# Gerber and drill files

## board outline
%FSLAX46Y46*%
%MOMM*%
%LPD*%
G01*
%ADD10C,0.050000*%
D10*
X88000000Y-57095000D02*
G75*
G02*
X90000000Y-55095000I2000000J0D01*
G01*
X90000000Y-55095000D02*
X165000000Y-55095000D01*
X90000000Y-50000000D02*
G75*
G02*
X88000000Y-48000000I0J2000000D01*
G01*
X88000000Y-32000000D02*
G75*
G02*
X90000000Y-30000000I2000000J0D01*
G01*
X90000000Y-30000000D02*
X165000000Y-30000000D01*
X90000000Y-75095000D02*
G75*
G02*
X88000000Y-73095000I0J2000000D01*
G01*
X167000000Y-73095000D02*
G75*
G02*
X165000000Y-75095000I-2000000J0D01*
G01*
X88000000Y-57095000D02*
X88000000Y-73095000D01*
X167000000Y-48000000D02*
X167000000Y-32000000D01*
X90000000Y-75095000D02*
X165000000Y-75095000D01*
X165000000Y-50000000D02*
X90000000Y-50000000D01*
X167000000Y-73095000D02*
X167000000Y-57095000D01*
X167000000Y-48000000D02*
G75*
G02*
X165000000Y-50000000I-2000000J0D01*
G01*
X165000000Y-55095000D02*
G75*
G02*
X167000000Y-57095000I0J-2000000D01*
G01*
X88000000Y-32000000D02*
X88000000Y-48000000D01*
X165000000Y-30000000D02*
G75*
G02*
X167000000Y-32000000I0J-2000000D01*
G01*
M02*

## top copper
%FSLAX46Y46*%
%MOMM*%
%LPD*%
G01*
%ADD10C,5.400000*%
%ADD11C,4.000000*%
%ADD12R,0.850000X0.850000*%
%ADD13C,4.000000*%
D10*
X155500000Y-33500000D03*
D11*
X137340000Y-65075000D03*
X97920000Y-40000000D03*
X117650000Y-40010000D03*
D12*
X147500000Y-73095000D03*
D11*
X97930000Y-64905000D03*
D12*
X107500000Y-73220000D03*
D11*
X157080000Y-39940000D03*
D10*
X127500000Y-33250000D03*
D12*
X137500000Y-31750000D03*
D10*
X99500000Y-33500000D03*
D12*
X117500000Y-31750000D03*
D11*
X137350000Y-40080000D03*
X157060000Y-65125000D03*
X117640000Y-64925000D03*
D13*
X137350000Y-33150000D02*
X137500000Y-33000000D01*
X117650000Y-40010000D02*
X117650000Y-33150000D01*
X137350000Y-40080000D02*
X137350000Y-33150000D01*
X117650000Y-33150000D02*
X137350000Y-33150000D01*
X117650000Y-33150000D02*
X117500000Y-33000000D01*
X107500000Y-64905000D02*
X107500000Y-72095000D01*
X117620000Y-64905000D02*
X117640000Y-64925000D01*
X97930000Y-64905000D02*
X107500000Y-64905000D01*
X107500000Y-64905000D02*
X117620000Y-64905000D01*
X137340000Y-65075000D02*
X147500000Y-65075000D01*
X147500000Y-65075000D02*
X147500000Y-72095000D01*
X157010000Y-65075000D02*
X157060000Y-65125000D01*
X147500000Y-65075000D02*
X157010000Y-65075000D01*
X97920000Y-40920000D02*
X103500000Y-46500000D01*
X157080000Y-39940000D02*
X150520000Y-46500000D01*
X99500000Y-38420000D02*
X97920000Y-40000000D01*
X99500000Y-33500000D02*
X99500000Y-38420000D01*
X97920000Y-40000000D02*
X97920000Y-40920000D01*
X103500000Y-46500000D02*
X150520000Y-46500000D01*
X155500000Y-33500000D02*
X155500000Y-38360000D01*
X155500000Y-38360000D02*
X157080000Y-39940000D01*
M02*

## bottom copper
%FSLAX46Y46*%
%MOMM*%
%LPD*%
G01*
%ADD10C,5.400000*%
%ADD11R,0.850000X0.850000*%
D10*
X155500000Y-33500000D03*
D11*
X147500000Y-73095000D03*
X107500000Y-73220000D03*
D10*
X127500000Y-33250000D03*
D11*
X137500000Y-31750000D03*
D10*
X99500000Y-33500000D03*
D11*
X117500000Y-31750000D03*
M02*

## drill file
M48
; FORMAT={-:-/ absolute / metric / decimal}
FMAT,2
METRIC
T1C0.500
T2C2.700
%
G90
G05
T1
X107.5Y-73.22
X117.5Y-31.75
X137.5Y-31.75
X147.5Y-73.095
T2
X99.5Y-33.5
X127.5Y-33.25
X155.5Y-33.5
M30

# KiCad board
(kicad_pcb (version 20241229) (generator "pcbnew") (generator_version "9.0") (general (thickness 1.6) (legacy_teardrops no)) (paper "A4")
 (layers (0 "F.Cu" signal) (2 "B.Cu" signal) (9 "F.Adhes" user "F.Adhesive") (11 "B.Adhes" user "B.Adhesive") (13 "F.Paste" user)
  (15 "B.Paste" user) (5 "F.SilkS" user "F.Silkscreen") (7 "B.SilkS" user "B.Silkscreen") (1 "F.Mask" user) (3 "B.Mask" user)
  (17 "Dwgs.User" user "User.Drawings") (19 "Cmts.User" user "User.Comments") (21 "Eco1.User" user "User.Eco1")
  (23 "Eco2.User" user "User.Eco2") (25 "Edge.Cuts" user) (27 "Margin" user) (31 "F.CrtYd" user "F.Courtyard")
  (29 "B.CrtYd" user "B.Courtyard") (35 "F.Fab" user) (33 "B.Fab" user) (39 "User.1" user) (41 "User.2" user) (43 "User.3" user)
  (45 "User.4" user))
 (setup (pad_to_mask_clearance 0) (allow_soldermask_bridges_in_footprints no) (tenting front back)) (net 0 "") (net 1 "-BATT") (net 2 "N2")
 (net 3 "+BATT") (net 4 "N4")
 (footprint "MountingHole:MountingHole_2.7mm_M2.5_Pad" (layer "F.Cu") (at 155.5 33.5)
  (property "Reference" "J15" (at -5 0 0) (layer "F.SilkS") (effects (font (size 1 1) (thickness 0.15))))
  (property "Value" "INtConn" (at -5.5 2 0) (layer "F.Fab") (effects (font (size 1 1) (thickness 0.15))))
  (pad "1" thru_hole circle (at 0 0) (size 5.4 5.4) (drill 2.7) (layers "*.Cu" "*.Mask") (remove_unused_layers no) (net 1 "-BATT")
   (zone_connect 2)))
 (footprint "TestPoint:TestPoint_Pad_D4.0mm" (layer "F.Cu") (at 137.34 65.075)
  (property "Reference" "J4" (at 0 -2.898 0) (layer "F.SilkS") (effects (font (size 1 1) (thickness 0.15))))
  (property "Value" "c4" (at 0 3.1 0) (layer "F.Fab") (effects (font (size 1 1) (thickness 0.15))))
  (pad "1" smd circle (at 0 0) (size 4 4) (layers "F.Cu" "F.Mask") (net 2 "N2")))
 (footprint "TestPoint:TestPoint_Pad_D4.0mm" (layer "F.Cu") (at 97.92 40)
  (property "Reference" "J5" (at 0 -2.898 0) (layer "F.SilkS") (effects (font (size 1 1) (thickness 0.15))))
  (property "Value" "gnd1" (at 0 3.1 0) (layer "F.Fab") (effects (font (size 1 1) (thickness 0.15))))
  (pad "1" smd circle (at 0 0) (size 4 4) (layers "F.Cu" "F.Mask") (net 1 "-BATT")))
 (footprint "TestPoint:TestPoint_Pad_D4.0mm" (layer "F.Cu") (at 117.65 40.01)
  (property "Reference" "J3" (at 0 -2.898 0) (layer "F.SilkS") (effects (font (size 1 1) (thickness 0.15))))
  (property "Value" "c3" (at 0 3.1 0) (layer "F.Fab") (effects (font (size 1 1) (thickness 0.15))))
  (pad "1" smd circle (at 0 0) (size 4 4) (layers "F.Cu" "F.Mask") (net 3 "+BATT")))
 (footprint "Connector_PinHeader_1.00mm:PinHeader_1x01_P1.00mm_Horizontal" (layer "F.Cu") (at 147.5 73.095 -90)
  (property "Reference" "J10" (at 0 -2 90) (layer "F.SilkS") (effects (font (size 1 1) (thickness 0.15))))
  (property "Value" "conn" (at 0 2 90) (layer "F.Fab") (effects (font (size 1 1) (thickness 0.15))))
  (pad "1" thru_hole rect (at 0 0 270) (size 0.85 0.85) (drill 0.5) (layers "*.Cu" "*.Mask") (remove_unused_layers no) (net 2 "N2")))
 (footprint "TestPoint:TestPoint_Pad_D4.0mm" (layer "F.Cu") (at 97.93 64.905)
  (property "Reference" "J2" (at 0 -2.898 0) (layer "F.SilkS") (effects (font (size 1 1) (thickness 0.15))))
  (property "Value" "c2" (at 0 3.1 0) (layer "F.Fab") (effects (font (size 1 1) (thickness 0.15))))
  (pad "1" smd circle (at 0 0) (size 4 4) (layers "F.Cu" "F.Mask") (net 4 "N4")))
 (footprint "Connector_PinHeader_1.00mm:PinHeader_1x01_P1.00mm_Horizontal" (layer "F.Cu") (at 107.5 73.22 -90)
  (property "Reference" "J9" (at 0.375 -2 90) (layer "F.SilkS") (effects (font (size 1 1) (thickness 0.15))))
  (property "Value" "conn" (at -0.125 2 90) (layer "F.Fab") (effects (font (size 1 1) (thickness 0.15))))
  (pad "1" thru_hole rect (at 0 0 270) (size 0.85 0.85) (drill 0.5) (layers "*.Cu" "*.Mask") (remove_unused_layers no) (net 4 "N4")))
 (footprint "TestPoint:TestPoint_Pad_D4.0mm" (layer "F.Cu") (at 157.08 39.94)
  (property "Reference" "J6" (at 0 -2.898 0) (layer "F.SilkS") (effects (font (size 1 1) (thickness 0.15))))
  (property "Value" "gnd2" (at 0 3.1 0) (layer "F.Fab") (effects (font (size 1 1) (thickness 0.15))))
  (pad "1" smd circle (at 0 0) (size 4 4) (layers "F.Cu" "F.Mask") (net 1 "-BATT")))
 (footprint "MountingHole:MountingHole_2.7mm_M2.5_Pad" (layer "F.Cu") (at 127.5 33.25)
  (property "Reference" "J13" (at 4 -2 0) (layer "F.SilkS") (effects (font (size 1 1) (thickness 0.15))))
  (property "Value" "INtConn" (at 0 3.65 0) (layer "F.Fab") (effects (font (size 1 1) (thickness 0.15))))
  (pad "1" thru_hole circle (at 0 0) (size 5.4 5.4) (drill 2.7) (layers "*.Cu" "*.Mask") (remove_unused_layers no) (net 3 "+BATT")
   (zone_connect 2)))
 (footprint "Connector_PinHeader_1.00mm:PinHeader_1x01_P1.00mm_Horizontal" (layer "F.Cu") (at 137.5 31.75 90)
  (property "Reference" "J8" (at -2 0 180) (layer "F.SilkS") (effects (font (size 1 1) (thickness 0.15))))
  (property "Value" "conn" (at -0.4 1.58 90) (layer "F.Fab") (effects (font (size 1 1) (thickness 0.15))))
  (pad "1" thru_hole rect (at 0 0 90) (size 0.85 0.85) (drill 0.5) (layers "*.Cu" "*.Mask") (remove_unused_layers no) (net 3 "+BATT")))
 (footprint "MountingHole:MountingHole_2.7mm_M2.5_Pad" (layer "F.Cu") (at 99.5 33.5)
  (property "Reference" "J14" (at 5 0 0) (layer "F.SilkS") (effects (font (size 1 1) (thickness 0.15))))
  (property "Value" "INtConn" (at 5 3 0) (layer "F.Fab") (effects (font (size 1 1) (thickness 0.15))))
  (pad "1" thru_hole circle (at 0 0) (size 5.4 5.4) (drill 2.7) (layers "*.Cu" "*.Mask") (remove_unused_layers no) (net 1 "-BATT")
   (zone_connect 2)))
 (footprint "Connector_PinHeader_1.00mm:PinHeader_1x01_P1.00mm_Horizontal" (layer "F.Cu") (at 117.5 31.75 90)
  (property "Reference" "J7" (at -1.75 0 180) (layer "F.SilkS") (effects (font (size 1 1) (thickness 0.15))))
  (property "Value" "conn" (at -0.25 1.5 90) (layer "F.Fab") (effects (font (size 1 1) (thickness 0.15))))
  (pad "1" thru_hole rect (at 0 0 90) (size 0.85 0.85) (drill 0.5) (layers "*.Cu" "*.Mask") (remove_unused_layers no) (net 3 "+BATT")))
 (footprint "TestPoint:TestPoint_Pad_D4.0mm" (layer "F.Cu") (at 137.35 40.08)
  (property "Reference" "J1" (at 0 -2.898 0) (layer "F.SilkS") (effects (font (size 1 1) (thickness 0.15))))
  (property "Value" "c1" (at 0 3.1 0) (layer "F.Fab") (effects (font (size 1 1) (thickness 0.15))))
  (pad "1" smd circle (at 0 0) (size 4 4) (layers "F.Cu" "F.Mask") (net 3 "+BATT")))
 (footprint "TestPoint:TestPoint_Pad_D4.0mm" (layer "F.Cu") (at 157.06 65.125)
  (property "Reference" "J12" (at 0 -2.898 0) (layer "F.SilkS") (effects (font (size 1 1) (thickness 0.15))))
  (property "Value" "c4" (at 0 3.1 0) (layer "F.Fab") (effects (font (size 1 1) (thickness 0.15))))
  (pad "1" smd circle (at 0 0) (size 4 4) (layers "F.Cu" "F.Mask") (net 2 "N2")))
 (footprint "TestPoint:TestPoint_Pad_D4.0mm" (layer "F.Cu") (at 117.64 64.925)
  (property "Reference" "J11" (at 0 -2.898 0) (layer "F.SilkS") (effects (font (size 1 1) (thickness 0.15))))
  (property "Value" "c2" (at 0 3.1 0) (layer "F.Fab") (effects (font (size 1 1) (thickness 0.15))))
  (pad "1" smd circle (at 0 0) (size 4 4) (layers "F.Cu" "F.Mask") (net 4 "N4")))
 (gr_arc (start 88 57.095) (mid 88.585786 55.680786) (end 90 55.095) (stroke (width 0.05) (type default)) (layer "Edge.Cuts"))
 (gr_line (start 90 55.095) (end 165 55.095) (stroke (width 0.05) (type default)) (layer "Edge.Cuts"))
 (gr_arc (start 90 50) (mid 88.585786 49.414214) (end 88 48) (stroke (width 0.05) (type default)) (layer "Edge.Cuts"))
 (gr_arc (start 88 32) (mid 88.585786 30.585786) (end 90 30) (stroke (width 0.05) (type default)) (layer "Edge.Cuts"))
 (gr_line (start 90 30) (end 165 30) (stroke (width 0.05) (type default)) (layer "Edge.Cuts"))
 (gr_arc (start 90 75.095) (mid 88.585786 74.509214) (end 88 73.095) (stroke (width 0.05) (type default)) (layer "Edge.Cuts"))
 (gr_arc (start 167 73.095) (mid 166.414214 74.509214) (end 165 75.095) (stroke (width 0.05) (type default)) (layer "Edge.Cuts"))
 (gr_line (start 88 57.095) (end 88 73.095) (stroke (width 0.05) (type default)) (layer "Edge.Cuts"))
 (gr_line (start 167 48) (end 167 32) (stroke (width 0.05) (type default)) (layer "Edge.Cuts"))
 (gr_line (start 90 75.095) (end 165 75.095) (stroke (width 0.05) (type default)) (layer "Edge.Cuts"))
 (gr_line (start 165 50) (end 90 50) (stroke (width 0.05) (type default)) (layer "Edge.Cuts"))
 (gr_line (start 167 73.095) (end 167 57.095) (stroke (width 0.05) (type default)) (layer "Edge.Cuts"))
 (gr_arc (start 167 48) (mid 166.414214 49.414214) (end 165 50) (stroke (width 0.05) (type default)) (layer "Edge.Cuts"))
 (gr_arc (start 165 55.095) (mid 166.414214 55.680786) (end 167 57.095) (stroke (width 0.05) (type default)) (layer "Edge.Cuts"))
 (gr_line (start 88 32) (end 88 48) (stroke (width 0.05) (type default)) (layer "Edge.Cuts"))
 (gr_arc (start 165 30) (mid 166.414214 30.585786) (end 167 32) (stroke (width 0.05) (type default)) (layer "Edge.Cuts"))
 (segment (start 137.35 33.15) (end 137.5 33) (width 4) (layer "F.Cu") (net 3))
 (segment (start 117.65 40.01) (end 117.65 33.15) (width 4) (layer "F.Cu") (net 3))
 (segment (start 137.35 40.08) (end 137.35 33.15) (width 4) (layer "F.Cu") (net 3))
 (segment (start 117.65 33.15) (end 137.35 33.15) (width 4) (layer "F.Cu") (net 3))
 (segment (start 117.65 33.15) (end 117.5 33) (width 4) (layer "F.Cu") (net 3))
 (segment (start 107.5 64.905) (end 107.5 72.095) (width 4) (layer "F.Cu") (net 4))
 (segment (start 117.62 64.905) (end 117.64 64.925) (width 4) (layer "F.Cu") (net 4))
 (segment (start 97.93 64.905) (end 107.5 64.905) (width 4) (layer "F.Cu") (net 4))
 (segment (start 107.5 64.905) (end 117.62 64.905) (width 4) (layer "F.Cu") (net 4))
 (segment (start 137.34 65.075) (end 147.5 65.075) (width 4) (layer "F.Cu") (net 2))
 (segment (start 147.5 65.075) (end 147.5 72.095) (width 4) (layer "F.Cu") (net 2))
 (segment (start 157.01 65.075) (end 157.06 65.125) (width 4) (layer "F.Cu") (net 2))
 (segment (start 147.5 65.075) (end 157.01 65.075) (width 4) (layer "F.Cu") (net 2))
 (segment (start 97.92 40.92) (end 103.5 46.5) (width 4) (layer "F.Cu") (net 1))
 (segment (start 157.08 39.94) (end 150.52 46.5) (width 4) (layer "F.Cu") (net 1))
 (segment (start 99.5 38.42) (end 97.92 40) (width 4) (layer "F.Cu") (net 1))
 (segment (start 99.5 33.5) (end 99.5 38.42) (width 4) (layer "F.Cu") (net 1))
 (segment (start 97.92 40) (end 97.92 40.92) (width 4) (layer "F.Cu") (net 1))
 (segment (start 103.5 46.5) (end 150.52 46.5) (width 4) (layer "F.Cu") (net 1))
 (segment (start 155.5 33.5) (end 155.5 38.36) (width 4) (layer "F.Cu") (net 1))
 (segment (start 155.5 38.36) (end 157.08 39.94) (width 4) (layer "F.Cu") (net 1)))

